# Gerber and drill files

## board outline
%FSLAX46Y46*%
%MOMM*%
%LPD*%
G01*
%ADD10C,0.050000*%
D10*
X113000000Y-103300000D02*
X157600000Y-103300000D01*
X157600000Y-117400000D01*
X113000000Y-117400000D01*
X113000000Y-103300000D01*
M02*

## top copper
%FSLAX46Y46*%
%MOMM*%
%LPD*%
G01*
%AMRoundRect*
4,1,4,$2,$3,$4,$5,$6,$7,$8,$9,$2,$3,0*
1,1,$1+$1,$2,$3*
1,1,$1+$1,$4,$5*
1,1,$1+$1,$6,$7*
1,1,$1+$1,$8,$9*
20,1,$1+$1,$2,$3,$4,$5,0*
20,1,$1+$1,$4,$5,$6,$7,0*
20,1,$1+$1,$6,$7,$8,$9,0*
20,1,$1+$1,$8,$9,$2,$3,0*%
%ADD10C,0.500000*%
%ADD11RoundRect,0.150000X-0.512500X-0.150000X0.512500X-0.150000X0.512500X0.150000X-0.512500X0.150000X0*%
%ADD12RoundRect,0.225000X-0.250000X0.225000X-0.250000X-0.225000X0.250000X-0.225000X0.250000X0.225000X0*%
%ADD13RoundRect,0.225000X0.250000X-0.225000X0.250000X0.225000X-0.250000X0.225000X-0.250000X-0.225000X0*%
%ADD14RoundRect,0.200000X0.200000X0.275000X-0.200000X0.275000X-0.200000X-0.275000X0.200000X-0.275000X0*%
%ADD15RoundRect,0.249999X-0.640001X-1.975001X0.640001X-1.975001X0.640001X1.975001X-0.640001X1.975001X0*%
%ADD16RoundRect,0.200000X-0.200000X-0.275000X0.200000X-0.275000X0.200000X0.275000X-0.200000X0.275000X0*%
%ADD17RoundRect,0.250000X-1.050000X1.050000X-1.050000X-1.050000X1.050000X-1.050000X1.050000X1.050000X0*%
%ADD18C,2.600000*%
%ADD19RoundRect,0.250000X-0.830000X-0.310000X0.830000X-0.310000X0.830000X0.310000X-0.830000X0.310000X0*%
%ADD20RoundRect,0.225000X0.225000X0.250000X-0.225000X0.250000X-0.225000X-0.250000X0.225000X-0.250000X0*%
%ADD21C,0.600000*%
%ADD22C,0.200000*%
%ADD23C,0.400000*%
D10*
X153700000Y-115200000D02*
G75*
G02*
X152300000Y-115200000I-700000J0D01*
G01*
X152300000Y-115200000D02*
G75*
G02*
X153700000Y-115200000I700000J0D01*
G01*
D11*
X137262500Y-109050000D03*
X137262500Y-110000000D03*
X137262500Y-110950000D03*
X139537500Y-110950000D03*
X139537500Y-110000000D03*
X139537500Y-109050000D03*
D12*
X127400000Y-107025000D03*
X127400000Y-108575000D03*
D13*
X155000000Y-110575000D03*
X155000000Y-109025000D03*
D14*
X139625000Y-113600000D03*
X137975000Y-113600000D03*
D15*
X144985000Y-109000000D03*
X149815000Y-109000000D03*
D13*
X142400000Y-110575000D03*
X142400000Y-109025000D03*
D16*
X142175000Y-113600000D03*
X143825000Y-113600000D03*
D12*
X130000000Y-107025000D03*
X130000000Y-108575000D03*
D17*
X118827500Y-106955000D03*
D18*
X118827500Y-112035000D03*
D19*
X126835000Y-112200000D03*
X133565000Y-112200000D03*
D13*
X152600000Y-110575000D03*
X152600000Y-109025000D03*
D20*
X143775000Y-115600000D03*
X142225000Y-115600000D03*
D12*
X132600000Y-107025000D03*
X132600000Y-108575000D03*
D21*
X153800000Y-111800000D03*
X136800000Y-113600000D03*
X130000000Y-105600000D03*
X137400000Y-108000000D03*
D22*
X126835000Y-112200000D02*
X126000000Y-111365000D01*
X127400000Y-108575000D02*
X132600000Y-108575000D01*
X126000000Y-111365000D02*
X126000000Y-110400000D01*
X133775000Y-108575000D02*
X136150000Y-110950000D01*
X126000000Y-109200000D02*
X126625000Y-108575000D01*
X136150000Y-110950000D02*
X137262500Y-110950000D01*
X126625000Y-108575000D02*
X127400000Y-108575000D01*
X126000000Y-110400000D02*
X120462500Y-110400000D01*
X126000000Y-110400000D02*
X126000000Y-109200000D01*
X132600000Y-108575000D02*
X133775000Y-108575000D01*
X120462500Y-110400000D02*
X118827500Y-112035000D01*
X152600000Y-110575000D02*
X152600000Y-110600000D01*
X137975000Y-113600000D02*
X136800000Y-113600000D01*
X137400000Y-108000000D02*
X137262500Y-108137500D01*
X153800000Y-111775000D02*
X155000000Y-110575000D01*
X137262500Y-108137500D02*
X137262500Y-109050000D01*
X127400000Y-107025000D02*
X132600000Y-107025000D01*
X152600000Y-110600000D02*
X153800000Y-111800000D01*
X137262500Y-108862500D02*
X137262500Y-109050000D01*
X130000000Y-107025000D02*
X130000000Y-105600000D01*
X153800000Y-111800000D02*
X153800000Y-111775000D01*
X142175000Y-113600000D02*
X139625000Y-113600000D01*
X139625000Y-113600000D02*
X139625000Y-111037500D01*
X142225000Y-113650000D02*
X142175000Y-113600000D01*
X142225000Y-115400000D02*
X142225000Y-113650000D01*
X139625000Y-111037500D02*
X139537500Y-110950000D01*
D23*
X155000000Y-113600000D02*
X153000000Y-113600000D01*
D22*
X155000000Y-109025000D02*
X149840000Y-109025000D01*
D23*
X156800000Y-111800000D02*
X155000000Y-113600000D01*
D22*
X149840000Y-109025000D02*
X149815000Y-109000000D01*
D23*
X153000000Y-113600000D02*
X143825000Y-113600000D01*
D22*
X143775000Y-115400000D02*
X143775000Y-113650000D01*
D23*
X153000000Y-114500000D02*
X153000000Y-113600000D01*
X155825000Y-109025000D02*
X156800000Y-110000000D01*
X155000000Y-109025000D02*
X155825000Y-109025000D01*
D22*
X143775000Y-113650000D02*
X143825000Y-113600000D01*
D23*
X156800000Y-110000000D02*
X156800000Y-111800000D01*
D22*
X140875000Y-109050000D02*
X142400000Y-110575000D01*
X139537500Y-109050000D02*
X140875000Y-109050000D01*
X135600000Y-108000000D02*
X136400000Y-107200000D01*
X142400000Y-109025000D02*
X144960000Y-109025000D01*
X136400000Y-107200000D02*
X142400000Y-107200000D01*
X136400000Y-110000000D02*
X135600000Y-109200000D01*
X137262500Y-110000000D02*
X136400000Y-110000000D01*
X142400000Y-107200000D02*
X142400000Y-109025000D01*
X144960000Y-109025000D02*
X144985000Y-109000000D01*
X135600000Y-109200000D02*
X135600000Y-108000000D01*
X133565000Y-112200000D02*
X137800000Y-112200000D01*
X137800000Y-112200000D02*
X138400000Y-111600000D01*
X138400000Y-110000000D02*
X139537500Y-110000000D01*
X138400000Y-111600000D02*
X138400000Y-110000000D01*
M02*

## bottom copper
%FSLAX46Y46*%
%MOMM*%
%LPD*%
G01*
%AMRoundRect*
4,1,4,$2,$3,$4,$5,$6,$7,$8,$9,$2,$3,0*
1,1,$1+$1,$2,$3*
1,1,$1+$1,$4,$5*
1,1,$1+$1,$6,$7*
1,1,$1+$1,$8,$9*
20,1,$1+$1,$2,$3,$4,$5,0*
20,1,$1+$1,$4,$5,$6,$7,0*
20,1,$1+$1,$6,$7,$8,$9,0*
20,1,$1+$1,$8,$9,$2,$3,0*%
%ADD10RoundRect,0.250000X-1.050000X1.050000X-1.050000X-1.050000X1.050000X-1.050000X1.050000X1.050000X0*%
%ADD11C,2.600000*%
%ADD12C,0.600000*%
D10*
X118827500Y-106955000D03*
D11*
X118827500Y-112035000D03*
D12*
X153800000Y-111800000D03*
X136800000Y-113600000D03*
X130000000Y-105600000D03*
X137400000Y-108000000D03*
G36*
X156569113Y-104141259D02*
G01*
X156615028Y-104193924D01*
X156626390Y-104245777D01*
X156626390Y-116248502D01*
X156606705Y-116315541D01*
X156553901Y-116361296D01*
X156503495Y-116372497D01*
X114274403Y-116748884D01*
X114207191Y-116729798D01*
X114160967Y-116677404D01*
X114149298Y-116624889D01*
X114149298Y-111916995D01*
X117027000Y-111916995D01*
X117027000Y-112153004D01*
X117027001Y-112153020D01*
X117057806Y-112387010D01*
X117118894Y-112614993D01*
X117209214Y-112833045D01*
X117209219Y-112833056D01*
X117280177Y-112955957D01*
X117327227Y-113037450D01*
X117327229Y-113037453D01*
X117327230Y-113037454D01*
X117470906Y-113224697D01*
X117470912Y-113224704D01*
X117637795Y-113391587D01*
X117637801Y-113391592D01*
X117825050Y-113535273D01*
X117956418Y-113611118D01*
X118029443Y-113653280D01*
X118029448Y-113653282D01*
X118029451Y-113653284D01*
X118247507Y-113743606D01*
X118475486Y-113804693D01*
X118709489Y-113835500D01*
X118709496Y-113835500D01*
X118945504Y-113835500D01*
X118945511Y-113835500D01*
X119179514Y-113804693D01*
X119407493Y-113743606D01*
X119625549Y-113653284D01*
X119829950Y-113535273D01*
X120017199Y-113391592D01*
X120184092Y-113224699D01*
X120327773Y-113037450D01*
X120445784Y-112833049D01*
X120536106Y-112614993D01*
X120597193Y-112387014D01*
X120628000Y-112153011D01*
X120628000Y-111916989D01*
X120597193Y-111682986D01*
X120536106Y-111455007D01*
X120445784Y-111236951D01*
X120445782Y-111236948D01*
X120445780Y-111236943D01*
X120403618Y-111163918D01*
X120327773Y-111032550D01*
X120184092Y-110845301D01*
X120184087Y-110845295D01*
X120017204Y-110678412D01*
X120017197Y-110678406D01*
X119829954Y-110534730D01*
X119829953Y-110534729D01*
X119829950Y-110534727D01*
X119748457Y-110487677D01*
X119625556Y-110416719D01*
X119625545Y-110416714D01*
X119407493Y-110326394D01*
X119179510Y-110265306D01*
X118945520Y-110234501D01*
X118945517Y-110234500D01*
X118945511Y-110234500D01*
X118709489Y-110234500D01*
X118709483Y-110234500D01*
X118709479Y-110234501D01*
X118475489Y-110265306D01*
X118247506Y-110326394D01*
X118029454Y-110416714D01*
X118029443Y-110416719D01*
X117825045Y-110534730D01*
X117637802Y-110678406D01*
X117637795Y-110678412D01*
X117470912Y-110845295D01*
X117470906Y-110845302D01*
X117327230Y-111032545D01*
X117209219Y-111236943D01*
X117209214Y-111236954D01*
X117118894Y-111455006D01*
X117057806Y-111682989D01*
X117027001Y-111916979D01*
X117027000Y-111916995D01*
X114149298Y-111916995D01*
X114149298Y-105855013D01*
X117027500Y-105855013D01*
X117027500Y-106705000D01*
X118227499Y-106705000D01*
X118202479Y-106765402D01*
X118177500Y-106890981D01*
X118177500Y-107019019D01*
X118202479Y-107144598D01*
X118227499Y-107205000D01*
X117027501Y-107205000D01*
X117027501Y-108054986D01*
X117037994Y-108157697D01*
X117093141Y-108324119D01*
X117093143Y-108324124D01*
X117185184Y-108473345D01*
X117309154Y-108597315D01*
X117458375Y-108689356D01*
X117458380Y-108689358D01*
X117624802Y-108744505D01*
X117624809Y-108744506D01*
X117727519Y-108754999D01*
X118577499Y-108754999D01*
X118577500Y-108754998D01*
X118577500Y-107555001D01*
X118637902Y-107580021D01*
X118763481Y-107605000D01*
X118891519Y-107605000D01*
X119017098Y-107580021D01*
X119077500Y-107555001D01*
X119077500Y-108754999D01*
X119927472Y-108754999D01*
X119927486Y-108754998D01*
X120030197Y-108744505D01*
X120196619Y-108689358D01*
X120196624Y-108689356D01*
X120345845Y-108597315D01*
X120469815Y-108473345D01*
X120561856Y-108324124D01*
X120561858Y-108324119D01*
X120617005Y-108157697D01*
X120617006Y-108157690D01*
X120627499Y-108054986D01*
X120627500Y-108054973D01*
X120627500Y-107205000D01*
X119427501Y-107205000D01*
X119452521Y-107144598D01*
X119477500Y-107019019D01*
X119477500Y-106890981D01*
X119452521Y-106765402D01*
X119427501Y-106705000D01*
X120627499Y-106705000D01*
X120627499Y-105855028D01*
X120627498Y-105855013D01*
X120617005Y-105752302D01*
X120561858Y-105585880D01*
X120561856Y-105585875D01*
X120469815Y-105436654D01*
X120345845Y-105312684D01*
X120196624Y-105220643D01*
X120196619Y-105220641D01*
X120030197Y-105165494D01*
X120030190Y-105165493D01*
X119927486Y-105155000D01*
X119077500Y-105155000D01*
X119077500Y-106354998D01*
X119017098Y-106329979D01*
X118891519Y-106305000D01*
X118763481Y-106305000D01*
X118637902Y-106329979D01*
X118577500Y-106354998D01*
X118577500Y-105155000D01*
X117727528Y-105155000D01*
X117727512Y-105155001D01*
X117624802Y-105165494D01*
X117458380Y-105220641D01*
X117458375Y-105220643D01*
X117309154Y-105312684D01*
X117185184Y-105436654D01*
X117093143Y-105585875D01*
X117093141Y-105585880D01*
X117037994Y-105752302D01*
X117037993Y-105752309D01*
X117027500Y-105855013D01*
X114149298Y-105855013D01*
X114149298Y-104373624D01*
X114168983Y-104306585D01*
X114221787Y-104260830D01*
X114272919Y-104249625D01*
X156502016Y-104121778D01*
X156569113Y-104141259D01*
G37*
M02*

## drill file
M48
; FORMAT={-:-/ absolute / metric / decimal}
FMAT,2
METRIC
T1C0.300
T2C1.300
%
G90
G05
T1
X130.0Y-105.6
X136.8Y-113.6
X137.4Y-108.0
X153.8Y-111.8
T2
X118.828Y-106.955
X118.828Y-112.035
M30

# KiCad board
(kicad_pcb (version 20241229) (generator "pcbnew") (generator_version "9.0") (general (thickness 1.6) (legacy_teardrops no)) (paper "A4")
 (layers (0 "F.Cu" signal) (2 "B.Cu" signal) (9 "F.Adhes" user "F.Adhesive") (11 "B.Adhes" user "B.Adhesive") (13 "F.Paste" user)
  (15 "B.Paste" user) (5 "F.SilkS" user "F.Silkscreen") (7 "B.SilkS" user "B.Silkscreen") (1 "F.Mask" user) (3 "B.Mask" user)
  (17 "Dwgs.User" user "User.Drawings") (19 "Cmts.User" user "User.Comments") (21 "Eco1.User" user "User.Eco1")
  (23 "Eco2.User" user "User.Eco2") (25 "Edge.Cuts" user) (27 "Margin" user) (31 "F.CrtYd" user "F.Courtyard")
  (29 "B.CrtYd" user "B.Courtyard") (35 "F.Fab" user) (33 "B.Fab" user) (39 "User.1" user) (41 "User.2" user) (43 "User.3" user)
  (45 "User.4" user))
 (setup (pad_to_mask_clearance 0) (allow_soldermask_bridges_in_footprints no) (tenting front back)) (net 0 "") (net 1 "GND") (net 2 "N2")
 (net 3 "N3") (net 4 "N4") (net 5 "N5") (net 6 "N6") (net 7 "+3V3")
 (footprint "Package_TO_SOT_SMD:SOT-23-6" (layer "F.Cu") (at 138.4 110)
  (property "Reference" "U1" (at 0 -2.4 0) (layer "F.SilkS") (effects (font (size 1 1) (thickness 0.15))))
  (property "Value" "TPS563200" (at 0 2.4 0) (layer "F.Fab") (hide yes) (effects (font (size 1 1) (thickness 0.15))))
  (pad "1" smd roundrect (at -1.1375 -0.95) (size 1.325 0.6) (layers "F.Cu" "F.Mask" "F.Paste") (roundrect_rratio 0.25) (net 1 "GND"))
  (pad "2" smd roundrect (at -1.1375 0) (size 1.325 0.6) (layers "F.Cu" "F.Mask" "F.Paste") (roundrect_rratio 0.25) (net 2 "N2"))
  (pad "3" smd roundrect (at -1.1375 0.95) (size 1.325 0.6) (layers "F.Cu" "F.Mask" "F.Paste") (roundrect_rratio 0.25) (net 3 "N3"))
  (pad "4" smd roundrect (at 1.1375 0.95) (size 1.325 0.6) (layers "F.Cu" "F.Mask" "F.Paste") (roundrect_rratio 0.25) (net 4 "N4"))
  (pad "5" smd roundrect (at 1.1375 0) (size 1.325 0.6) (layers "F.Cu" "F.Mask" "F.Paste") (roundrect_rratio 0.25) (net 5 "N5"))
  (pad "6" smd roundrect (at 1.1375 -0.95) (size 1.325 0.6) (layers "F.Cu" "F.Mask" "F.Paste") (roundrect_rratio 0.25) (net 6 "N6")))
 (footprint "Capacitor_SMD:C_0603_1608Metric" (layer "F.Cu") (at 127.4 107.8 -90)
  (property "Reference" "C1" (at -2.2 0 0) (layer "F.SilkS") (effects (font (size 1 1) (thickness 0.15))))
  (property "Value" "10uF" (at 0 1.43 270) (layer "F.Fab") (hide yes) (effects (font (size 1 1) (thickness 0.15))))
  (pad "1" smd roundrect (at -0.775 0 270) (size 0.9 0.95) (layers "F.Cu" "F.Mask" "F.Paste") (roundrect_rratio 0.25) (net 1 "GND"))
  (pad "2" smd roundrect (at 0.775 0 270) (size 0.9 0.95) (layers "F.Cu" "F.Mask" "F.Paste") (roundrect_rratio 0.25) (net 3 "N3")))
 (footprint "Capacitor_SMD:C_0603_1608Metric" (layer "F.Cu") (at 155 109.8 90)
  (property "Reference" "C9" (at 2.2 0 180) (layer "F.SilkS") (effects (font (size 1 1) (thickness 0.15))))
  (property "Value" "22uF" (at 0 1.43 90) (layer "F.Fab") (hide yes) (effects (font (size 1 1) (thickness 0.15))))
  (pad "1" smd roundrect (at -0.775 0 90) (size 0.9 0.95) (layers "F.Cu" "F.Mask" "F.Paste") (roundrect_rratio 0.25) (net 1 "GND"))
  (pad "2" smd roundrect (at 0.775 0 90) (size 0.9 0.95) (layers "F.Cu" "F.Mask" "F.Paste") (roundrect_rratio 0.25) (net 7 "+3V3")))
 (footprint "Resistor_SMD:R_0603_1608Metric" (layer "F.Cu") (at 138.8 113.6 180)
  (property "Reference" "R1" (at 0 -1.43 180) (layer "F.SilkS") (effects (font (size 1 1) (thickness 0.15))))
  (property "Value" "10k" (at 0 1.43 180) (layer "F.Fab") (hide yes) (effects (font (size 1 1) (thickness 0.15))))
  (pad "1" smd roundrect (at -0.825 0 180) (size 0.8 0.95) (layers "F.Cu" "F.Mask" "F.Paste") (roundrect_rratio 0.25) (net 4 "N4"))
  (pad "2" smd roundrect (at 0.825 0 180) (size 0.8 0.95) (layers "F.Cu" "F.Mask" "F.Paste") (roundrect_rratio 0.25) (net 1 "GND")))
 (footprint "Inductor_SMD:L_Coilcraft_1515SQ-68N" (layer "F.Cu") (at 147.4 109)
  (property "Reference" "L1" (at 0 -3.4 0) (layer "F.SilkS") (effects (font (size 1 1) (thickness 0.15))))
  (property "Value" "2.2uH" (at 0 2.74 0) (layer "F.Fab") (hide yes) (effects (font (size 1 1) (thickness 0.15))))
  (pad "1" smd roundrect (at -2.415 0) (size 1.78 4.45) (layers "F.Cu" "F.Mask" "F.Paste") (roundrect_rratio 0.140449) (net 2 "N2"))
  (pad "2" smd roundrect (at 2.415 0) (size 1.78 4.45) (layers "F.Cu" "F.Mask" "F.Paste") (roundrect_rratio 0.140449) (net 7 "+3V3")))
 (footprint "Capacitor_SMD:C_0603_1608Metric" (layer "F.Cu") (at 142.4 109.8 90)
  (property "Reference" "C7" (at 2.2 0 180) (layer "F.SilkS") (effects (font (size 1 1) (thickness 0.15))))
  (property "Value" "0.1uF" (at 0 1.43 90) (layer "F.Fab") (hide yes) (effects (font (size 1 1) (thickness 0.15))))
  (pad "1" smd roundrect (at -0.775 0 90) (size 0.9 0.95) (layers "F.Cu" "F.Mask" "F.Paste") (roundrect_rratio 0.25) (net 6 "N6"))
  (pad "2" smd roundrect (at 0.775 0 90) (size 0.9 0.95) (layers "F.Cu" "F.Mask" "F.Paste") (roundrect_rratio 0.25) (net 2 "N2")))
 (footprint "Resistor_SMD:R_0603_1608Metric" (layer "F.Cu") (at 143 113.6)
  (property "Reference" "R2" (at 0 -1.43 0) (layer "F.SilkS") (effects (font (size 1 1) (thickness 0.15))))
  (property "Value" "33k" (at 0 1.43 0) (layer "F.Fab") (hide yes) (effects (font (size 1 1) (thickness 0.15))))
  (pad "1" smd roundrect (at -0.825 0) (size 0.8 0.95) (layers "F.Cu" "F.Mask" "F.Paste") (roundrect_rratio 0.25) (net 4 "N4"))
  (pad "2" smd roundrect (at 0.825 0) (size 0.8 0.95) (layers "F.Cu" "F.Mask" "F.Paste") (roundrect_rratio 0.25) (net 7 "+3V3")))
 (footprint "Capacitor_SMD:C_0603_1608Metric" (layer "F.Cu") (at 130 107.8 -90)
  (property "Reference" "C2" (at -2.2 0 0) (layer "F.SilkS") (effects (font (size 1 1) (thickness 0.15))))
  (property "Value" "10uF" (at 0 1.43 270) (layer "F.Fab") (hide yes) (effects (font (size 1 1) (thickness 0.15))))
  (pad "1" smd roundrect (at -0.775 0 270) (size 0.9 0.95) (layers "F.Cu" "F.Mask" "F.Paste") (roundrect_rratio 0.25) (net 1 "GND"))
  (pad "2" smd roundrect (at 0.775 0 270) (size 0.9 0.95) (layers "F.Cu" "F.Mask" "F.Paste") (roundrect_rratio 0.25) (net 3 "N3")))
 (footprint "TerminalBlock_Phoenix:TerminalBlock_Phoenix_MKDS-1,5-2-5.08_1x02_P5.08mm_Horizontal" (layer "F.Cu") (at 118.8275 106.955 -90)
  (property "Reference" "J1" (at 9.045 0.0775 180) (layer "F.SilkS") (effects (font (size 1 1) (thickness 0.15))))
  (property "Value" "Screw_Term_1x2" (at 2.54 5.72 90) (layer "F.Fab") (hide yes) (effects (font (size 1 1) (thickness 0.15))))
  (pad "1" thru_hole roundrect (at 0 0 270) (size 2.6 2.6) (drill 1.3) (layers "*.Cu" "*.Mask") (remove_unused_layers no)
   (roundrect_rratio 0.096154) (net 1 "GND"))
  (pad "2" thru_hole circle (at 5.08 0 270) (size 2.6 2.6) (drill 1.3) (layers "*.Cu" "*.Mask") (remove_unused_layers no) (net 3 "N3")))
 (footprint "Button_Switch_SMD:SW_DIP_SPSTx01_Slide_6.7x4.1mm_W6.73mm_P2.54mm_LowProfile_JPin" (layer "F.Cu") (at 130.2 112.2)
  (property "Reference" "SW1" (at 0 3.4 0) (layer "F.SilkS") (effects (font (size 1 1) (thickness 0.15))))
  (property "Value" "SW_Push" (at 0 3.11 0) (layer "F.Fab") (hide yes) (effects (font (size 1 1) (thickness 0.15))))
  (pad "1" smd roundrect (at -3.365 0) (size 2.16 1.12) (layers "F.Cu" "F.Mask" "F.Paste") (roundrect_rratio 0.223214) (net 3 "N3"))
  (pad "2" smd roundrect (at 3.365 0) (size 2.16 1.12) (layers "F.Cu" "F.Mask" "F.Paste") (roundrect_rratio 0.223214) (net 5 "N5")))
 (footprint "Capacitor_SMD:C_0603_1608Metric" (layer "F.Cu") (at 152.6 109.8 90)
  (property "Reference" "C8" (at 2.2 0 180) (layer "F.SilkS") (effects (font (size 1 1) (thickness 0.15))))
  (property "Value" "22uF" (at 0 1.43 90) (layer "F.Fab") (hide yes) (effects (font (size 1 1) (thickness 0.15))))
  (pad "1" smd roundrect (at -0.775 0 90) (size 0.9 0.95) (layers "F.Cu" "F.Mask" "F.Paste") (roundrect_rratio 0.25) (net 1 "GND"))
  (pad "2" smd roundrect (at 0.775 0 90) (size 0.9 0.95) (layers "F.Cu" "F.Mask" "F.Paste") (roundrect_rratio 0.25) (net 7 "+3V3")))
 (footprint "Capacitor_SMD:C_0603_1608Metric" (layer "F.Cu") (at 143 115.6 180)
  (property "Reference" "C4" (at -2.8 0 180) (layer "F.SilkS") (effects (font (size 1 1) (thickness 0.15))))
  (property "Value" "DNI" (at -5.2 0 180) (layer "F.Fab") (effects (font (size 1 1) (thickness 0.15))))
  (pad "1" smd roundrect (at -0.775 0 180) (size 0.9 0.95) (layers "F.Cu" "F.Mask" "F.Paste") (roundrect_rratio 0.25) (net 7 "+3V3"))
  (pad "2" smd roundrect (at 0.775 0 180) (size 0.9 0.95) (layers "F.Cu" "F.Mask" "F.Paste") (roundrect_rratio 0.25) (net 4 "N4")))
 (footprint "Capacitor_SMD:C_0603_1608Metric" (layer "F.Cu") (at 132.6 107.8 -90)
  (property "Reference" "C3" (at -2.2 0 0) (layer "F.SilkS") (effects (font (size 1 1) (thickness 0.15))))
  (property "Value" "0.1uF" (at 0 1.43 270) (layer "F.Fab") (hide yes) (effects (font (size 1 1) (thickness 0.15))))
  (pad "1" smd roundrect (at -0.775 0 270) (size 0.9 0.95) (layers "F.Cu" "F.Mask" "F.Paste") (roundrect_rratio 0.25) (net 1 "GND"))
  (pad "2" smd roundrect (at 0.775 0 270) (size 0.9 0.95) (layers "F.Cu" "F.Mask" "F.Paste") (roundrect_rratio 0.25) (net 3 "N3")))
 (gr_circle (center 153 115.2) (end 153.7 115.2) (stroke (width 0.5) (type solid)) (fill no) (layer "F.Cu") (net 7))
 (gr_rect (start 113 103.3) (end 157.6 117.4) (stroke (width 0.05) (type default)) (fill no) (layer "Edge.Cuts"))
 (segment (start 126.835 112.2) (end 126 111.365) (width 0.2) (layer "F.Cu") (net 3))
 (segment (start 127.4 108.575) (end 132.6 108.575) (width 0.2) (layer "F.Cu") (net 3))
 (segment (start 126 111.365) (end 126 110.4) (width 0.2) (layer "F.Cu") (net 3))
 (segment (start 133.775 108.575) (end 136.15 110.95) (width 0.2) (layer "F.Cu") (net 3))
 (segment (start 126 109.2) (end 126.625 108.575) (width 0.2) (layer "F.Cu") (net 3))
 (segment (start 136.15 110.95) (end 137.2625 110.95) (width 0.2) (layer "F.Cu") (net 3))
 (segment (start 126.625 108.575) (end 127.4 108.575) (width 0.2) (layer "F.Cu") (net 3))
 (segment (start 126 110.4) (end 120.4625 110.4) (width 0.2) (layer "F.Cu") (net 3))
 (segment (start 126 110.4) (end 126 109.2) (width 0.2) (layer "F.Cu") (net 3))
 (segment (start 132.6 108.575) (end 133.775 108.575) (width 0.2) (layer "F.Cu") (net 3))
 (segment (start 120.4625 110.4) (end 118.8275 112.035) (width 0.2) (layer "F.Cu") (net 3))
 (segment (start 152.6 110.575) (end 152.6 110.6) (width 0.2) (layer "F.Cu") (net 1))
 (segment (start 137.975 113.6) (end 136.8 113.6) (width 0.2) (layer "F.Cu") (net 1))
 (segment (start 137.4 108) (end 137.2625 108.1375) (width 0.2) (layer "F.Cu") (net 1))
 (segment (start 153.8 111.775) (end 155 110.575) (width 0.2) (layer "F.Cu") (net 1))
 (segment (start 137.2625 108.1375) (end 137.2625 109.05) (width 0.2) (layer "F.Cu") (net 1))
 (segment (start 127.4 107.025) (end 132.6 107.025) (width 0.2) (layer "F.Cu") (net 1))
 (segment (start 152.6 110.6) (end 153.8 111.8) (width 0.2) (layer "F.Cu") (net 1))
 (segment (start 137.2625 108.8625) (end 137.2625 109.05) (width 0.2) (layer "F.Cu") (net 1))
 (segment (start 130 107.025) (end 130 105.6) (width 0.2) (layer "F.Cu") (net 1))
 (segment (start 153.8 111.8) (end 153.8 111.775) (width 0.2) (layer "F.Cu") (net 1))
 (via (at 153.8 111.8) (size 0.6) (drill 0.3) (layers "F.Cu" "B.Cu") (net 1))
 (via (at 136.8 113.6) (size 0.6) (drill 0.3) (layers "F.Cu" "B.Cu") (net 1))
 (via (at 130 105.6) (size 0.6) (drill 0.3) (layers "F.Cu" "B.Cu") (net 1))
 (via (at 137.4 108) (size 0.6) (drill 0.3) (layers "F.Cu" "B.Cu") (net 1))
 (segment (start 142.175 113.6) (end 139.625 113.6) (width 0.2) (layer "F.Cu") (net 4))
 (segment (start 139.625 113.6) (end 139.625 111.0375) (width 0.2) (layer "F.Cu") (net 4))
 (segment (start 142.225 113.65) (end 142.175 113.6) (width 0.2) (layer "F.Cu") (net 4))
 (segment (start 142.225 115.4) (end 142.225 113.65) (width 0.2) (layer "F.Cu") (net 4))
 (segment (start 139.625 111.0375) (end 139.5375 110.95) (width 0.2) (layer "F.Cu") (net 4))
 (segment (start 155 113.6) (end 153 113.6) (width 0.4) (layer "F.Cu") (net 7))
 (segment (start 155 109.025) (end 149.84 109.025) (width 0.2) (layer "F.Cu") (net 7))
 (segment (start 156.8 111.8) (end 155 113.6) (width 0.4) (layer "F.Cu") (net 7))
 (segment (start 149.84 109.025) (end 149.815 109) (width 0.2) (layer "F.Cu") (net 7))
 (segment (start 153 113.6) (end 143.825 113.6) (width 0.4) (layer "F.Cu") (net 7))
 (segment (start 143.775 115.4) (end 143.775 113.65) (width 0.2) (layer "F.Cu") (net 7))
 (segment (start 153 114.5) (end 153 113.6) (width 0.4) (layer "F.Cu") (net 7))
 (segment (start 155.825 109.025) (end 156.8 110) (width 0.4) (layer "F.Cu") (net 7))
 (segment (start 155 109.025) (end 155.825 109.025) (width 0.4) (layer "F.Cu") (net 7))
 (segment (start 143.775 113.65) (end 143.825 113.6) (width 0.2) (layer "F.Cu") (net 7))
 (segment (start 156.8 110) (end 156.8 111.8) (width 0.4) (layer "F.Cu") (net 7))
 (segment (start 140.875 109.05) (end 142.4 110.575) (width 0.2) (layer "F.Cu") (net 6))
 (segment (start 139.5375 109.05) (end 140.875 109.05) (width 0.2) (layer "F.Cu") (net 6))
 (segment (start 135.6 108) (end 136.4 107.2) (width 0.2) (layer "F.Cu") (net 2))
 (segment (start 142.4 109.025) (end 144.96 109.025) (width 0.2) (layer "F.Cu") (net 2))
 (segment (start 136.4 107.2) (end 142.4 107.2) (width 0.2) (layer "F.Cu") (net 2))
 (segment (start 136.4 110) (end 135.6 109.2) (width 0.2) (layer "F.Cu") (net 2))
 (segment (start 137.2625 110) (end 136.4 110) (width 0.2) (layer "F.Cu") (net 2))
 (segment (start 142.4 107.2) (end 142.4 109.025) (width 0.2) (layer "F.Cu") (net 2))
 (segment (start 144.96 109.025) (end 144.985 109) (width 0.2) (layer "F.Cu") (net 2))
 (segment (start 135.6 109.2) (end 135.6 108) (width 0.2) (layer "F.Cu") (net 2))
 (segment (start 133.565 112.2) (end 137.8 112.2) (width 0.2) (layer "F.Cu") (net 5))
 (segment (start 137.8 112.2) (end 138.4 111.6) (width 0.2) (layer "F.Cu") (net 5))
 (segment (start 138.4 110) (end 139.5375 110) (width 0.2) (layer "F.Cu") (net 5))
 (segment (start 138.4 111.6) (end 138.4 110) (width 0.2) (layer "F.Cu") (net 5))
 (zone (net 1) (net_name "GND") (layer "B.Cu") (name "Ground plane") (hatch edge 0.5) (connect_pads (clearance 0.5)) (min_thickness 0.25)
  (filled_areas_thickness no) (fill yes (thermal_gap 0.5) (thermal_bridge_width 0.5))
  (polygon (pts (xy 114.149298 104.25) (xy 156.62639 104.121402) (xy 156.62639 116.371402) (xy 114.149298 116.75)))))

